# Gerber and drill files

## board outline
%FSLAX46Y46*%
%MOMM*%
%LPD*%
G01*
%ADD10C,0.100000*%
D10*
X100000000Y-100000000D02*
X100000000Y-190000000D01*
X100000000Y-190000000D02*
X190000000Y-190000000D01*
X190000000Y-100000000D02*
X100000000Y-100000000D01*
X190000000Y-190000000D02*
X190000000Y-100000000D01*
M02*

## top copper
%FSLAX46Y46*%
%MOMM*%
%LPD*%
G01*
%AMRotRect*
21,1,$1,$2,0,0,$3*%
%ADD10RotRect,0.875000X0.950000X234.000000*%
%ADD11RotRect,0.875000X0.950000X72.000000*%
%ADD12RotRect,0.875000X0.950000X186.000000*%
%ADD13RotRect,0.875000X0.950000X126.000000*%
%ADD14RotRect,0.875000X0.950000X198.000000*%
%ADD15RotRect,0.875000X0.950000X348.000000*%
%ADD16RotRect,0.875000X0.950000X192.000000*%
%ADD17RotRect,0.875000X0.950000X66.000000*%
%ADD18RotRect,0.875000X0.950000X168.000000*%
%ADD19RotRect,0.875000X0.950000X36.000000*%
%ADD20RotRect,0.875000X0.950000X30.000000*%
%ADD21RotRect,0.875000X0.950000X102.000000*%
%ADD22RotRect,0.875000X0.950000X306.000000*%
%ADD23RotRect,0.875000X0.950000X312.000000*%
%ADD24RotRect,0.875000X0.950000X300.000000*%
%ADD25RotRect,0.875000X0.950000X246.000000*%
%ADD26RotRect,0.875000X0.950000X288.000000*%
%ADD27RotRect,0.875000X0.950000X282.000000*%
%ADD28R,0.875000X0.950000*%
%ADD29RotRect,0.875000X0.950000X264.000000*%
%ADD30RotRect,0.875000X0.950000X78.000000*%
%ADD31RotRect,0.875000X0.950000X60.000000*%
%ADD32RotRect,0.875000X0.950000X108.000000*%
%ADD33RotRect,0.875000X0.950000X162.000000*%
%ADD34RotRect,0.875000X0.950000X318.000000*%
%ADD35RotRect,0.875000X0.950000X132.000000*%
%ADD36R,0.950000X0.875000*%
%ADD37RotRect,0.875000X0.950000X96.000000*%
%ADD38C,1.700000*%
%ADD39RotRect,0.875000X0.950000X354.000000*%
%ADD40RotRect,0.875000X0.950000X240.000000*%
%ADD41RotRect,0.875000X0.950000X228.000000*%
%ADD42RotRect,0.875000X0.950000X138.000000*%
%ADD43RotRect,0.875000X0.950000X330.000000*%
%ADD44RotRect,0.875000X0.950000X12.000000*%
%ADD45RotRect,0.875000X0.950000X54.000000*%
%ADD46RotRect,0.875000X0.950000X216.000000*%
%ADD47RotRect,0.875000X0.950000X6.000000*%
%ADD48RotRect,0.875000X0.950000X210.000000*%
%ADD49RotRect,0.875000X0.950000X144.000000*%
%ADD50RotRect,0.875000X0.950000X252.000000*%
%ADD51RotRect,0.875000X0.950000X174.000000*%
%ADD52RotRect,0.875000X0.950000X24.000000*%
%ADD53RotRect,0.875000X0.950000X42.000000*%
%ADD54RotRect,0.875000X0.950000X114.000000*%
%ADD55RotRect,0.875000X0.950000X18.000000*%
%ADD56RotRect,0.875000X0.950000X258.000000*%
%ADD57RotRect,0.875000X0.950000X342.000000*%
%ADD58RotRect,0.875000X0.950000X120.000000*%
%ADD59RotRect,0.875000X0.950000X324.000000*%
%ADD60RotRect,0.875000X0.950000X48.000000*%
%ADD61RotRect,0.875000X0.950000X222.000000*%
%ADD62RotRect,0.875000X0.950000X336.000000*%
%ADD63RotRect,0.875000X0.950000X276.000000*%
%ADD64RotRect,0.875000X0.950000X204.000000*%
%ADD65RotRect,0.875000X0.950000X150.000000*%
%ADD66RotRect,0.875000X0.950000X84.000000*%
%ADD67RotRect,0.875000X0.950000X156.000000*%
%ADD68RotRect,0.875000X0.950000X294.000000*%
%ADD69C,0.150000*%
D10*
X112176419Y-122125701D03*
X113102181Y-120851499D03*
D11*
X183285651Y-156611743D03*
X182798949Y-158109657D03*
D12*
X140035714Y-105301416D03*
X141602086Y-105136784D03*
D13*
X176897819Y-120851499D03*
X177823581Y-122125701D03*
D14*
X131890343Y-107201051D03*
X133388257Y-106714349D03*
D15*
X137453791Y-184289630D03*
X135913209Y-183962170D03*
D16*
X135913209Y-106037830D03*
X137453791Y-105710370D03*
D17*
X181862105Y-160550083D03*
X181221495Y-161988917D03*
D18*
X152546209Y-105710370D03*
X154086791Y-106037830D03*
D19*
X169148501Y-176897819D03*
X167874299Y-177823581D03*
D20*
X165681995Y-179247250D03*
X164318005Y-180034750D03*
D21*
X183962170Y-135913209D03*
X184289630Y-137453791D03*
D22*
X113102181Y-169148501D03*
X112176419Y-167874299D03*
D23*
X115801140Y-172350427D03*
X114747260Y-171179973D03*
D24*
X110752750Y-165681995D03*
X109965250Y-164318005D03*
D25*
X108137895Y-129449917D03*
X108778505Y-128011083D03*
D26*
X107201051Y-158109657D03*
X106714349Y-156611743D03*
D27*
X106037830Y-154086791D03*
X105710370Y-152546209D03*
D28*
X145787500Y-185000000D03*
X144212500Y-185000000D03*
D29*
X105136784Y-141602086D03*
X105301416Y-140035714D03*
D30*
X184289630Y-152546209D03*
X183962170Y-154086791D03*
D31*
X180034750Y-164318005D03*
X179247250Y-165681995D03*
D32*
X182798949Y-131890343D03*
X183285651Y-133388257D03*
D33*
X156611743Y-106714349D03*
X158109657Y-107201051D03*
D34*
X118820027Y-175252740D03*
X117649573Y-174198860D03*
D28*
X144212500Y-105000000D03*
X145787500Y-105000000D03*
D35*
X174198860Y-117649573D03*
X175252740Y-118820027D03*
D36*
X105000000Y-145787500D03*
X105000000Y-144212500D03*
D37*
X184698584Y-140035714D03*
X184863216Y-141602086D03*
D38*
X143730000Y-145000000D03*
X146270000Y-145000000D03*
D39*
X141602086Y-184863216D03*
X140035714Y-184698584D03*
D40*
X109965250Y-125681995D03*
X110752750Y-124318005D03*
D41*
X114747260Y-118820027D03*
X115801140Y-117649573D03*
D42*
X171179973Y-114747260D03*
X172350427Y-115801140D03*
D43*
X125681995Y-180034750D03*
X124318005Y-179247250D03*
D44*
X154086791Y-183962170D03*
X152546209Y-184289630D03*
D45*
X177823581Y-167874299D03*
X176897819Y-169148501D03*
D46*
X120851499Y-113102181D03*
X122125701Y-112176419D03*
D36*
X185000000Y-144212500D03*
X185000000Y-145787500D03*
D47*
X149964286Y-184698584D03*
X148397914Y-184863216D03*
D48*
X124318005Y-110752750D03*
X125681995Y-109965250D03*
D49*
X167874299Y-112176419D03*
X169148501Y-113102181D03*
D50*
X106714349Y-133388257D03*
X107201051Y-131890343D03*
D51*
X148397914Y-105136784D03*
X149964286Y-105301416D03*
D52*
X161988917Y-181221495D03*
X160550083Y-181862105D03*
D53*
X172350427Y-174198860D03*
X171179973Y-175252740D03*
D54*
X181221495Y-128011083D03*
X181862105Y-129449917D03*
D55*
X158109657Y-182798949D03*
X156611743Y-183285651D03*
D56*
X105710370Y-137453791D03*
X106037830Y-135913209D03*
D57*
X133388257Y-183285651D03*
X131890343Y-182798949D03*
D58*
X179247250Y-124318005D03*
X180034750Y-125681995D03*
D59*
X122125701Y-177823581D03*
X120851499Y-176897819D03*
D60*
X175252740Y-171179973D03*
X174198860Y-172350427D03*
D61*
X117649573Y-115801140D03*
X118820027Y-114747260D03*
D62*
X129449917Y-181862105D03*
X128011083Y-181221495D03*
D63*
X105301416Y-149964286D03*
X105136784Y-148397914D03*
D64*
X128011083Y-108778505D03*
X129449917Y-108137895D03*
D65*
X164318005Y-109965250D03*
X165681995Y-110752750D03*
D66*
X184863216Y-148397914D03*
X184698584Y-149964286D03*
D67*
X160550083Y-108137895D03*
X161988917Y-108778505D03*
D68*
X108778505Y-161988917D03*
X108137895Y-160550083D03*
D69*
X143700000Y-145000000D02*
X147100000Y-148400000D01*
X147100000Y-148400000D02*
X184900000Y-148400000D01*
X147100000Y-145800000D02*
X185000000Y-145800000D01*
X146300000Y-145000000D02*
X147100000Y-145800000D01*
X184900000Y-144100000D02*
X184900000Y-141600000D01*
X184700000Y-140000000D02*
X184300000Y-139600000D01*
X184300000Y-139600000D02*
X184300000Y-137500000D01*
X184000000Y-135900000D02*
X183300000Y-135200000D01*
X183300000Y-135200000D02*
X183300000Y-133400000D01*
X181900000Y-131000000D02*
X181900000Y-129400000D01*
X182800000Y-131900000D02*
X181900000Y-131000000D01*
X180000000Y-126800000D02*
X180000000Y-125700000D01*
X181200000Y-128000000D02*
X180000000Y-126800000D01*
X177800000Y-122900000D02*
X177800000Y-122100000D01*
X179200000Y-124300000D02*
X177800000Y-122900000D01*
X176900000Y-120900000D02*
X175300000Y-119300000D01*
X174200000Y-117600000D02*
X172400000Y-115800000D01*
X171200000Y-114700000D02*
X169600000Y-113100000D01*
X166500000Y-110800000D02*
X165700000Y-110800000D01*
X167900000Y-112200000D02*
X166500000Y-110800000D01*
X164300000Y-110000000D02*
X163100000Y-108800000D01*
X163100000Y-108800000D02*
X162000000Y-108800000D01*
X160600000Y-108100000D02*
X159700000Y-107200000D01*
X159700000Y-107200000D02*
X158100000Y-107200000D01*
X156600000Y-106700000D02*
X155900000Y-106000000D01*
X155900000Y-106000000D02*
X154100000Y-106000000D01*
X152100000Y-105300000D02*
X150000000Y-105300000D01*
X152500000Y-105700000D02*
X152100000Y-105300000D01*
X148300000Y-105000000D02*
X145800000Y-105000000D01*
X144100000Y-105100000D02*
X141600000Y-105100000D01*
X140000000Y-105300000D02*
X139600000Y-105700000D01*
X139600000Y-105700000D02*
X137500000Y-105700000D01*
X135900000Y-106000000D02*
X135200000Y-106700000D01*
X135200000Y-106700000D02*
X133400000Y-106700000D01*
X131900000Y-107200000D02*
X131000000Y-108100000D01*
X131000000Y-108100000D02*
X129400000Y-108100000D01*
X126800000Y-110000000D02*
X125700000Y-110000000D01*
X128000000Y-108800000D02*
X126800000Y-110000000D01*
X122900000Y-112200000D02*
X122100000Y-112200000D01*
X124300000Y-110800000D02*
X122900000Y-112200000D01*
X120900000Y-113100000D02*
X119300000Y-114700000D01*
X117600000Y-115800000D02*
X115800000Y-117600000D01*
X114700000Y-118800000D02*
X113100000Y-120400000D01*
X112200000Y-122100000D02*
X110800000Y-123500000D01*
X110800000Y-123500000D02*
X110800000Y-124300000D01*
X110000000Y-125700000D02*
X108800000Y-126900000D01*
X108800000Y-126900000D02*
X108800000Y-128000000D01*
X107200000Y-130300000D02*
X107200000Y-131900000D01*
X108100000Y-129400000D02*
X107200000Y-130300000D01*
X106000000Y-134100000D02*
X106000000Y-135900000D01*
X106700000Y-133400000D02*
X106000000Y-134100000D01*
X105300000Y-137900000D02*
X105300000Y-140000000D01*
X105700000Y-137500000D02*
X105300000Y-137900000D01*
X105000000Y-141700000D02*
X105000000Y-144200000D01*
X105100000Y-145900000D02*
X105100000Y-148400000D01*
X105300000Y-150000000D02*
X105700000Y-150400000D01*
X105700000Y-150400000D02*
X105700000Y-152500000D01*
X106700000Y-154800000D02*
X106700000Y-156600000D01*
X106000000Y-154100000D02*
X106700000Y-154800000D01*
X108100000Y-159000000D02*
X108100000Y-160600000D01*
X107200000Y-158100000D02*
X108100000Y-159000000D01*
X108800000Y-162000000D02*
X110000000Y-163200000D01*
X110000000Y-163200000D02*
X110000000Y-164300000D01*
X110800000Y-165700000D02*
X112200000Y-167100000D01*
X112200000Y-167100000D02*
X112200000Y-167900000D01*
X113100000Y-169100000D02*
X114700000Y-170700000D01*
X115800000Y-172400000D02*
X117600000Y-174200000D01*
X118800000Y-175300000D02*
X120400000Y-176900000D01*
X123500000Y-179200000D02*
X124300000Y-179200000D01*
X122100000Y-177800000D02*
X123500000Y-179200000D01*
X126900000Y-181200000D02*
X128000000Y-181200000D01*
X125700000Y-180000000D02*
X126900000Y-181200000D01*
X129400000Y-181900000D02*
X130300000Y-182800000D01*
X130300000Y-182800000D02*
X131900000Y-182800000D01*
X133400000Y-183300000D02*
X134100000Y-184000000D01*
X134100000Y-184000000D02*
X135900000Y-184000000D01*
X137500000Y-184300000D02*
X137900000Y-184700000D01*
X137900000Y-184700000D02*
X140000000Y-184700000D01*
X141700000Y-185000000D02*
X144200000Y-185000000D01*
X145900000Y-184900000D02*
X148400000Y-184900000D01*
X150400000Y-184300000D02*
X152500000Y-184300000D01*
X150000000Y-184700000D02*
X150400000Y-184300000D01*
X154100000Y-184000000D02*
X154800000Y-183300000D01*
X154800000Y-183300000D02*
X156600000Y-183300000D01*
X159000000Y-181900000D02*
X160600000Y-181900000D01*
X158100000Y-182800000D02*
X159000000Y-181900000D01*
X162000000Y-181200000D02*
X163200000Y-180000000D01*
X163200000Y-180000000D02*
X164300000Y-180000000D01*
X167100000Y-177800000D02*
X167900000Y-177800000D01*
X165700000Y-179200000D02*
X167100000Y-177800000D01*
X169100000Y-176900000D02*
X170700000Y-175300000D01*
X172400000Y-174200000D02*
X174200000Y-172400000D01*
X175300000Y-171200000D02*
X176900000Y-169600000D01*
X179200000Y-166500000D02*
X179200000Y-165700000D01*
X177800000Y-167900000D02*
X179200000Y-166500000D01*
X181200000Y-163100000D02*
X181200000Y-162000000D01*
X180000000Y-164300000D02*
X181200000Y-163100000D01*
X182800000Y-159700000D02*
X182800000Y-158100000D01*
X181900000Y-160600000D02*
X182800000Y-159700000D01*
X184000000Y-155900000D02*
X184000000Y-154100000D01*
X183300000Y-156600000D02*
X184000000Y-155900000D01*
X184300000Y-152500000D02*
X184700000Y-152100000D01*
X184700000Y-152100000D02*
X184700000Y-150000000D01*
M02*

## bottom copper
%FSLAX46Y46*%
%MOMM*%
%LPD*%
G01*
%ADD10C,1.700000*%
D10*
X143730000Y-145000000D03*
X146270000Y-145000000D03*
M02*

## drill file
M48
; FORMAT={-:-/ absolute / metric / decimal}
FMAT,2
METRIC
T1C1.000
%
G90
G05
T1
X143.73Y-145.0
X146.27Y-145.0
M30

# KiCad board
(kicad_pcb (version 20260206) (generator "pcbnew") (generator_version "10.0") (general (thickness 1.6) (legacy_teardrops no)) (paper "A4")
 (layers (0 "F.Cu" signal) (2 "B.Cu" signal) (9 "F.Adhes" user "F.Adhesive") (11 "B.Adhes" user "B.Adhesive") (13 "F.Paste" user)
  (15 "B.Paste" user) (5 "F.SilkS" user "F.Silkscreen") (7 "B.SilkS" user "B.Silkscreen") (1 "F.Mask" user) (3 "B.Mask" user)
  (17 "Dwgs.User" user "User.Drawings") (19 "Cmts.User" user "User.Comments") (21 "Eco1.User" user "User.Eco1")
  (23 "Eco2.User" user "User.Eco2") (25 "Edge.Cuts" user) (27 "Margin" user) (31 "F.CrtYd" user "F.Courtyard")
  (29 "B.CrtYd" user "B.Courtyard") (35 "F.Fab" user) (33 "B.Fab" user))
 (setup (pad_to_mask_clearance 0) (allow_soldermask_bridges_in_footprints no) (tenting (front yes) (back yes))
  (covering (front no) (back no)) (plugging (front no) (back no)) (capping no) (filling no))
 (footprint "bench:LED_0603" (layer "F.Cu") (at 112.6393 121.4886 -126)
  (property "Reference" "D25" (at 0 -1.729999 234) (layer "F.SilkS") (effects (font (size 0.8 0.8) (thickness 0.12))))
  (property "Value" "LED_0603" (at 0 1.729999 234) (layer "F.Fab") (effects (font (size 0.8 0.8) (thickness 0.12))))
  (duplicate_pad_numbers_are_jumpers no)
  (pad "A" smd rect (at 0.7875 0 234) (size 0.875 0.95) (layers "F.Cu" "F.Mask" "F.Paste") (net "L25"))
  (pad "K" smd rect (at -0.7875 0 234) (size 0.875 0.95) (layers "F.Cu" "F.Mask" "F.Paste") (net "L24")))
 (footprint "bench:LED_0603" (layer "F.Cu") (at 183.0423 157.3607 72)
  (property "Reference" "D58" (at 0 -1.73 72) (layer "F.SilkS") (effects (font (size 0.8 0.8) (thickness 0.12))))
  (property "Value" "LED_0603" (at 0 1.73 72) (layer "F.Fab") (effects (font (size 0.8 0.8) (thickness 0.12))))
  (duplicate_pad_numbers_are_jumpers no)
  (pad "A" smd rect (at 0.7875 0 72) (size 0.875 0.95) (layers "F.Cu" "F.Mask" "F.Paste") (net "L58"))
  (pad "K" smd rect (at -0.7875 0 72) (size 0.875 0.95) (layers "F.Cu" "F.Mask" "F.Paste") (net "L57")))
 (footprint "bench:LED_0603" (layer "F.Cu") (at 140.8189 105.2191 -174)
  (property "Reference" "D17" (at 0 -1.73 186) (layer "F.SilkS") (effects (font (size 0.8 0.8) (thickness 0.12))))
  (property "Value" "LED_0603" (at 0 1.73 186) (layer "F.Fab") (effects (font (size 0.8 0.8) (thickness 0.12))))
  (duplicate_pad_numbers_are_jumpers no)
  (pad "A" smd rect (at 0.7875 0 186) (size 0.875 0.95) (layers "F.Cu" "F.Mask" "F.Paste") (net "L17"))
  (pad "K" smd rect (at -0.7875 0 186) (size 0.875 0.95) (layers "F.Cu" "F.Mask" "F.Paste") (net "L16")))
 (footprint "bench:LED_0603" (layer "F.Cu") (at 177.3607 121.4886 126)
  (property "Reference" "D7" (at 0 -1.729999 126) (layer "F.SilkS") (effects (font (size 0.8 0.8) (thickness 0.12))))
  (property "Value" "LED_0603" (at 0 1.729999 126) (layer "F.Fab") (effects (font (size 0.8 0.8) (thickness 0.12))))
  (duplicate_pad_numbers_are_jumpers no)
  (pad "A" smd rect (at 0.7875 0 126) (size 0.875 0.95) (layers "F.Cu" "F.Mask" "F.Paste") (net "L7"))
  (pad "K" smd rect (at -0.7875 0 126) (size 0.875 0.95) (layers "F.Cu" "F.Mask" "F.Paste") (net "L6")))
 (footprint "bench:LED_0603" (layer "F.Cu") (at 132.6393 106.9577 -162)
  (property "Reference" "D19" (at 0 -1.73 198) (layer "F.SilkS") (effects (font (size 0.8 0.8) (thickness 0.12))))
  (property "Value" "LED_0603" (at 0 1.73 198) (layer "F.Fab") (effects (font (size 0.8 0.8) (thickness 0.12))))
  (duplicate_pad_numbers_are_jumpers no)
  (pad "A" smd rect (at 0.7875 0 198) (size 0.875 0.95) (layers "F.Cu" "F.Mask" "F.Paste") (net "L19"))
  (pad "K" smd rect (at -0.7875 0 198) (size 0.875 0.95) (layers "F.Cu" "F.Mask" "F.Paste") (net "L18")))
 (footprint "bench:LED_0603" (layer "F.Cu") (at 136.6835 184.1259 -12)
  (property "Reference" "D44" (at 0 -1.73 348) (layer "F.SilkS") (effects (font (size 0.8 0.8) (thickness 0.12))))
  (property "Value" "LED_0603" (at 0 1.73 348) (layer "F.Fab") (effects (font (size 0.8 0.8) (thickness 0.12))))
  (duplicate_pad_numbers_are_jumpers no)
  (pad "A" smd rect (at 0.7875 0 348) (size 0.875 0.95) (layers "F.Cu" "F.Mask" "F.Paste") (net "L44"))
  (pad "K" smd rect (at -0.7875 0 348) (size 0.875 0.95) (layers "F.Cu" "F.Mask" "F.Paste") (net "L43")))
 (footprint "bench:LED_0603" (layer "F.Cu") (at 136.6835 105.8741 -168)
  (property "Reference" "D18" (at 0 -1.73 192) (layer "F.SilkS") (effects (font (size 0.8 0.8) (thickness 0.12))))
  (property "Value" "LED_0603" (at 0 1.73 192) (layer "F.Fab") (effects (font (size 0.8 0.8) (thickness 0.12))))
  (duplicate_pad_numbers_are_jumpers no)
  (pad "A" smd rect (at 0.7875 0 192) (size 0.875 0.95) (layers "F.Cu" "F.Mask" "F.Paste") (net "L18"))
  (pad "K" smd rect (at -0.7875 0 192) (size 0.875 0.95) (layers "F.Cu" "F.Mask" "F.Paste") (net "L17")))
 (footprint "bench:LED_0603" (layer "F.Cu") (at 181.5418 161.2695 66)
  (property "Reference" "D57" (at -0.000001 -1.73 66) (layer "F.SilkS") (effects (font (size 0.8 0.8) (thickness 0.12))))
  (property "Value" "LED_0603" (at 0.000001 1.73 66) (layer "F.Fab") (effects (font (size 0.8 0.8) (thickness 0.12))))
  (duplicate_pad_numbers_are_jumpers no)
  (pad "A" smd rect (at 0.7875 0 66) (size 0.875 0.95) (layers "F.Cu" "F.Mask" "F.Paste") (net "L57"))
  (pad "K" smd rect (at -0.7875 0 66) (size 0.875 0.95) (layers "F.Cu" "F.Mask" "F.Paste") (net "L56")))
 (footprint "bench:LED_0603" (layer "F.Cu") (at 153.3165 105.8741 168)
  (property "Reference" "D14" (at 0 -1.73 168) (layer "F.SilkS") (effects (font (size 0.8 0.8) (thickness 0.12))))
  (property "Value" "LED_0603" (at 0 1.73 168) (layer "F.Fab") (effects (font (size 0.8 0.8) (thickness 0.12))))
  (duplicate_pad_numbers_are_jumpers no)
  (pad "A" smd rect (at 0.7875 0 168) (size 0.875 0.95) (layers "F.Cu" "F.Mask" "F.Paste") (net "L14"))
  (pad "K" smd rect (at -0.7875 0 168) (size 0.875 0.95) (layers "F.Cu" "F.Mask" "F.Paste") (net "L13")))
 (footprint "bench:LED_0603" (layer "F.Cu") (at 168.5114 177.3607 36)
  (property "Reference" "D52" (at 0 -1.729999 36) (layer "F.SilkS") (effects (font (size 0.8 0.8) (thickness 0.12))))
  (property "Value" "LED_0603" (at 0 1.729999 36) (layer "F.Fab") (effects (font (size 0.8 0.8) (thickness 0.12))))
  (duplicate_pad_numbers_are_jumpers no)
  (pad "A" smd rect (at 0.7875 0 36) (size 0.875 0.95) (layers "F.Cu" "F.Mask" "F.Paste") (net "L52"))
  (pad "K" smd rect (at -0.7875 0 36) (size 0.875 0.95) (layers "F.Cu" "F.Mask" "F.Paste") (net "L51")))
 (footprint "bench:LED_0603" (layer "F.Cu") (at 165 179.641 30)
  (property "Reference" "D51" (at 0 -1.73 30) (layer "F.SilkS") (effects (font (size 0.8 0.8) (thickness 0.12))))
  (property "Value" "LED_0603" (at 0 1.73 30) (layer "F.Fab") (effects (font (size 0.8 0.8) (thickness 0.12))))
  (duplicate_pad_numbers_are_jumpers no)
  (pad "A" smd rect (at 0.7875 0 30) (size 0.875 0.95) (layers "F.Cu" "F.Mask" "F.Paste") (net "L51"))
  (pad "K" smd rect (at -0.7875 0 30) (size 0.875 0.95) (layers "F.Cu" "F.Mask" "F.Paste") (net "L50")))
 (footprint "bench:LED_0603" (layer "F.Cu") (at 184.1259 136.6835 102)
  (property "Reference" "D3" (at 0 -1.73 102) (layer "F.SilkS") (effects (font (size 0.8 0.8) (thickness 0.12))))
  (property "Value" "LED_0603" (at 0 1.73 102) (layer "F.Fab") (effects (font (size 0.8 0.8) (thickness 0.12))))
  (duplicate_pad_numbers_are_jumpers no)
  (pad "A" smd rect (at 0.7875 0 102) (size 0.875 0.95) (layers "F.Cu" "F.Mask" "F.Paste") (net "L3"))
  (pad "K" smd rect (at -0.7875 0 102) (size 0.875 0.95) (layers "F.Cu" "F.Mask" "F.Paste") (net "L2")))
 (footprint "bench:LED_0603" (layer "F.Cu") (at 112.6393 168.5114 -54)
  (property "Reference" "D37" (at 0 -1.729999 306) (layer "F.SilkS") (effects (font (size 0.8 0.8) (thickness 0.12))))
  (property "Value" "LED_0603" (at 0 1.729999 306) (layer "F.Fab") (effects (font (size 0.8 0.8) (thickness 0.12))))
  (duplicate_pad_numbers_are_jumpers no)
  (pad "A" smd rect (at 0.7875 0 306) (size 0.875 0.95) (layers "F.Cu" "F.Mask" "F.Paste") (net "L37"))
  (pad "K" smd rect (at -0.7875 0 306) (size 0.875 0.95) (layers "F.Cu" "F.Mask" "F.Paste") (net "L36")))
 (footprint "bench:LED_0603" (layer "F.Cu") (at 115.2742 171.7652 -48)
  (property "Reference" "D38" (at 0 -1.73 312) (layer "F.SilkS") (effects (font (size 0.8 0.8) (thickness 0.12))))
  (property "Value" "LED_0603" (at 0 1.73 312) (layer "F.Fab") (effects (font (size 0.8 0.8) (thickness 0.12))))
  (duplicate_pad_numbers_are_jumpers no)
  (pad "A" smd rect (at 0.7875 0.000001 312) (size 0.875 0.95) (layers "F.Cu" "F.Mask" "F.Paste") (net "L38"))
  (pad "K" smd rect (at -0.7875 -0.000001 312) (size 0.875 0.95) (layers "F.Cu" "F.Mask" "F.Paste") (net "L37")))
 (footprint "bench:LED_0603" (layer "F.Cu") (at 110.359 165 -60)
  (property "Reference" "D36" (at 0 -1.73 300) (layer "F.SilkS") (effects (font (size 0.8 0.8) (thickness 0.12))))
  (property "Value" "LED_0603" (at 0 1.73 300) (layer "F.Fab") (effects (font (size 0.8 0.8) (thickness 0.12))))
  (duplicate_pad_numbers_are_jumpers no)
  (pad "A" smd rect (at 0.7875 0 300) (size 0.875 0.95) (layers "F.Cu" "F.Mask" "F.Paste") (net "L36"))
  (pad "K" smd rect (at -0.7875 0 300) (size 0.875 0.95) (layers "F.Cu" "F.Mask" "F.Paste") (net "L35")))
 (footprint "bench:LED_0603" (layer "F.Cu") (at 108.4582 128.7305 -114)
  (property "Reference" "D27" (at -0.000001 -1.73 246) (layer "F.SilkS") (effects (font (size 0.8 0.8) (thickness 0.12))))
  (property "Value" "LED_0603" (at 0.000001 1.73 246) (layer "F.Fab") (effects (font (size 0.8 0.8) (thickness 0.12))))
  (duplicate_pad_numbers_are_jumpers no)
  (pad "A" smd rect (at 0.7875 0 246) (size 0.875 0.95) (layers "F.Cu" "F.Mask" "F.Paste") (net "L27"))
  (pad "K" smd rect (at -0.7875 0 246) (size 0.875 0.95) (layers "F.Cu" "F.Mask" "F.Paste") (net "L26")))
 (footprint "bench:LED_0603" (layer "F.Cu") (at 106.9577 157.3607 -72)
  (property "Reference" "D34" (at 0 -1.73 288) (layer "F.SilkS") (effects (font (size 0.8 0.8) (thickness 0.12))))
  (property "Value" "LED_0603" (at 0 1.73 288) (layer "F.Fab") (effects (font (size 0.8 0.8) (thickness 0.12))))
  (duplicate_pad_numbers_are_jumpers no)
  (pad "A" smd rect (at 0.7875 0 288) (size 0.875 0.95) (layers "F.Cu" "F.Mask" "F.Paste") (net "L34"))
  (pad "K" smd rect (at -0.7875 0 288) (size 0.875 0.95) (layers "F.Cu" "F.Mask" "F.Paste") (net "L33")))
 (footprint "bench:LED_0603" (layer "F.Cu") (at 105.8741 153.3165 -78)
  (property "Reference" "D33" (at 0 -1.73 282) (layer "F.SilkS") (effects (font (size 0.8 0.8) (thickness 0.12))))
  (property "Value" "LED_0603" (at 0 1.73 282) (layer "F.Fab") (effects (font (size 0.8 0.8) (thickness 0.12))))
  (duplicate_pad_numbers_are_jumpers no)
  (pad "A" smd rect (at 0.7875 0 282) (size 0.875 0.95) (layers "F.Cu" "F.Mask" "F.Paste") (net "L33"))
  (pad "K" smd rect (at -0.7875 0 282) (size 0.875 0.95) (layers "F.Cu" "F.Mask" "F.Paste") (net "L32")))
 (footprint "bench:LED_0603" (layer "F.Cu") (at 145 185)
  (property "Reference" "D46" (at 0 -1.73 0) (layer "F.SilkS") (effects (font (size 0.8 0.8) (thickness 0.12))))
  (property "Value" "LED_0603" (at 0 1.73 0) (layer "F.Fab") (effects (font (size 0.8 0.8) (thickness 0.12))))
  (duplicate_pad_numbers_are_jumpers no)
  (pad "A" smd rect (at 0.7875 0) (size 0.875 0.95) (layers "F.Cu" "F.Mask" "F.Paste") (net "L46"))
  (pad "K" smd rect (at -0.7875 0) (size 0.875 0.95) (layers "F.Cu" "F.Mask" "F.Paste") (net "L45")))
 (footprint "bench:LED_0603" (layer "F.Cu") (at 105.2191 140.8189 -96)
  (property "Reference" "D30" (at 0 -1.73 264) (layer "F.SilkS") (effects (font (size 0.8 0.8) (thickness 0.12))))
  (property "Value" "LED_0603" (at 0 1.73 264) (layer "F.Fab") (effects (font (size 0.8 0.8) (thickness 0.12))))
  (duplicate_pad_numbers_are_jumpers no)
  (pad "A" smd rect (at 0.7875 0 264) (size 0.875 0.95) (layers "F.Cu" "F.Mask" "F.Paste") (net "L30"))
  (pad "K" smd rect (at -0.7875 0 264) (size 0.875 0.95) (layers "F.Cu" "F.Mask" "F.Paste") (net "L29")))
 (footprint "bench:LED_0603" (layer "F.Cu") (at 184.1259 153.3165 78)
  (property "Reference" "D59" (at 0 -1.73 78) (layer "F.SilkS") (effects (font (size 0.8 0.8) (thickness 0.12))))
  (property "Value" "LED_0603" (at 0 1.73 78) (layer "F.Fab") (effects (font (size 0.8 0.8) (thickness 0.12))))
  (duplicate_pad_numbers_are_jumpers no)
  (pad "A" smd rect (at 0.7875 0 78) (size 0.875 0.95) (layers "F.Cu" "F.Mask" "F.Paste") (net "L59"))
  (pad "K" smd rect (at -0.7875 0 78) (size 0.875 0.95) (layers "F.Cu" "F.Mask" "F.Paste") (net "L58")))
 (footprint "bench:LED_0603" (layer "F.Cu") (at 179.641 165 60)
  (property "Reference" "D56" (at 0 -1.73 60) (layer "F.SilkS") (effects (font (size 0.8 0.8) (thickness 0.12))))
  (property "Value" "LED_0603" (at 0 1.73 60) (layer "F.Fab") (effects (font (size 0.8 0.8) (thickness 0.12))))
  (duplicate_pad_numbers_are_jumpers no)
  (pad "A" smd rect (at 0.7875 0 60) (size 0.875 0.95) (layers "F.Cu" "F.Mask" "F.Paste") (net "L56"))
  (pad "K" smd rect (at -0.7875 0 60) (size 0.875 0.95) (layers "F.Cu" "F.Mask" "F.Paste") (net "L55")))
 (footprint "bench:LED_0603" (layer "F.Cu") (at 183.0423 132.6393 108)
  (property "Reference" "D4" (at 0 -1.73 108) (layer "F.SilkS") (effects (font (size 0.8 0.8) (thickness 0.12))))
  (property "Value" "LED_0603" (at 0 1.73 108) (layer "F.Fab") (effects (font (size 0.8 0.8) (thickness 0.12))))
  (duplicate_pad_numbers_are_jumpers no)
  (pad "A" smd rect (at 0.7875 0 108) (size 0.875 0.95) (layers "F.Cu" "F.Mask" "F.Paste") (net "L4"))
  (pad "K" smd rect (at -0.7875 0 108) (size 0.875 0.95) (layers "F.Cu" "F.Mask" "F.Paste") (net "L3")))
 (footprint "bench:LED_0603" (layer "F.Cu") (at 157.3607 106.9577 162)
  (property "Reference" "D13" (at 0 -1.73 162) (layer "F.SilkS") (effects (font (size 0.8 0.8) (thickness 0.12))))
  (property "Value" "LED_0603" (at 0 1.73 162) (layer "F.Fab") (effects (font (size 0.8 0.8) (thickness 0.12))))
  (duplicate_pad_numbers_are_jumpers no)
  (pad "A" smd rect (at 0.7875 0 162) (size 0.875 0.95) (layers "F.Cu" "F.Mask" "F.Paste") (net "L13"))
  (pad "K" smd rect (at -0.7875 0 162) (size 0.875 0.95) (layers "F.Cu" "F.Mask" "F.Paste") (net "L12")))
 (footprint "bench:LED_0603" (layer "F.Cu") (at 118.2348 174.7258 -42)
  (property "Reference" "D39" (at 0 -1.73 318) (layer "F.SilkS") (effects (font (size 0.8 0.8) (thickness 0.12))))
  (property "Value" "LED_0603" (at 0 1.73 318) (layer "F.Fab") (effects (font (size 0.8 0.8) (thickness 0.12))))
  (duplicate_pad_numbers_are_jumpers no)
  (pad "A" smd rect (at 0.7875 -0.000001 318) (size 0.875 0.95) (layers "F.Cu" "F.Mask" "F.Paste") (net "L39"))
  (pad "K" smd rect (at -0.7875 0.000001 318) (size 0.875 0.95) (layers "F.Cu" "F.Mask" "F.Paste") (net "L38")))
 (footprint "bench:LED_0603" (layer "F.Cu") (at 145 105 180)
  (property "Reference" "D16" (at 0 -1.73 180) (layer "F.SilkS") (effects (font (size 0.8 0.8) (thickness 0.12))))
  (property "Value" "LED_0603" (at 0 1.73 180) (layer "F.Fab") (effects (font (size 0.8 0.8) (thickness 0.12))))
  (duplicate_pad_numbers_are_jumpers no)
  (pad "A" smd rect (at 0.7875 0 180) (size 0.875 0.95) (layers "F.Cu" "F.Mask" "F.Paste") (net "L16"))
  (pad "K" smd rect (at -0.7875 0 180) (size 0.875 0.95) (layers "F.Cu" "F.Mask" "F.Paste") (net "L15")))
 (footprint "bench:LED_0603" (layer "F.Cu") (at 174.7258 118.2348 132)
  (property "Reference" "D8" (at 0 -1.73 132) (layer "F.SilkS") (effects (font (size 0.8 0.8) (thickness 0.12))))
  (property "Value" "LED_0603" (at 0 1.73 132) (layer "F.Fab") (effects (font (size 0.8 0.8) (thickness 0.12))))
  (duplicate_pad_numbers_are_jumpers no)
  (pad "A" smd rect (at 0.7875 0.000001 132) (size 0.875 0.95) (layers "F.Cu" "F.Mask" "F.Paste") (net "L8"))
  (pad "K" smd rect (at -0.7875 -0.000001 132) (size 0.875 0.95) (layers "F.Cu" "F.Mask" "F.Paste") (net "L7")))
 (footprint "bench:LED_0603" (layer "F.Cu") (at 105 145 -90)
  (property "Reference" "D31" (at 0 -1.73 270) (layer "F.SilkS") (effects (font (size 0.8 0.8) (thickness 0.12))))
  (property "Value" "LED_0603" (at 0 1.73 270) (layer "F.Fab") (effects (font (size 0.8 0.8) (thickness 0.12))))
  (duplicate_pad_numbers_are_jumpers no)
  (pad "A" smd rect (at 0.7875 0 270) (size 0.875 0.95) (layers "F.Cu" "F.Mask" "F.Paste") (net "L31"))
  (pad "K" smd rect (at -0.7875 0 270) (size 0.875 0.95) (layers "F.Cu" "F.Mask" "F.Paste") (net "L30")))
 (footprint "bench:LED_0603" (layer "F.Cu") (at 184.7809 140.8189 96)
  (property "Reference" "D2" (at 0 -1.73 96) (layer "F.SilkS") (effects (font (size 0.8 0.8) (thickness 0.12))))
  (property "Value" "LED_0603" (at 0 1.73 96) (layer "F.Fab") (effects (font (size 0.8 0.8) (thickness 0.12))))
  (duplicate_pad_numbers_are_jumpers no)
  (pad "A" smd rect (at 0.7875 0 96) (size 0.875 0.95) (layers "F.Cu" "F.Mask" "F.Paste") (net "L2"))
  (pad "K" smd rect (at -0.7875 0 96) (size 0.875 0.95) (layers "F.Cu" "F.Mask" "F.Paste") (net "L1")))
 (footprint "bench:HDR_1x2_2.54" (layer "F.Cu") (at 143.73 145)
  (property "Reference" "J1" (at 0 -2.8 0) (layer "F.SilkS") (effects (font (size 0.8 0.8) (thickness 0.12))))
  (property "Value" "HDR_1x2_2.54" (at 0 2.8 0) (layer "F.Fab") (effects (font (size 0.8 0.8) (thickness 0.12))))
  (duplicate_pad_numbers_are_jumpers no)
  (pad "1" thru_hole circle (at 0 0) (size 1.7 1.7) (drill 1) (layers "*.Cu" "*.Mask") (remove_unused_layers no) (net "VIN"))
  (pad "2" thru_hole circle (at 2.54 0) (size 1.7 1.7) (drill 1) (layers "*.Cu" "*.Mask") (remove_unused_layers no) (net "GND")))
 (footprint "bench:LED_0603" (layer "F.Cu") (at 140.8189 184.7809 -6)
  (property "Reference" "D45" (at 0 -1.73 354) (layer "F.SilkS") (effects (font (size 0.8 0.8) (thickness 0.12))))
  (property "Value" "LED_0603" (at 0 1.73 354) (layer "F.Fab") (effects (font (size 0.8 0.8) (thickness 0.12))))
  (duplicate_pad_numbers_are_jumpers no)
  (pad "A" smd rect (at 0.7875 0 354) (size 0.875 0.95) (layers "F.Cu" "F.Mask" "F.Paste") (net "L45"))
  (pad "K" smd rect (at -0.7875 0 354) (size 0.875 0.95) (layers "F.Cu" "F.Mask" "F.Paste") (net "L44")))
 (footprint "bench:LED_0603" (layer "F.Cu") (at 110.359 125 -120)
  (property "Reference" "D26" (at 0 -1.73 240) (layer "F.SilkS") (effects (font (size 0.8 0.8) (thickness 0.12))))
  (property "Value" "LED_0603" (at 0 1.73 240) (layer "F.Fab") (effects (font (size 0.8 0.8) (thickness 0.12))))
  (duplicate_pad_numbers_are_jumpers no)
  (pad "A" smd rect (at 0.7875 0 240) (size 0.875 0.95) (layers "F.Cu" "F.Mask" "F.Paste") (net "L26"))
  (pad "K" smd rect (at -0.7875 0 240) (size 0.875 0.95) (layers "F.Cu" "F.Mask" "F.Paste") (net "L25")))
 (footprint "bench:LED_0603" (layer "F.Cu") (at 115.2742 118.2348 -132)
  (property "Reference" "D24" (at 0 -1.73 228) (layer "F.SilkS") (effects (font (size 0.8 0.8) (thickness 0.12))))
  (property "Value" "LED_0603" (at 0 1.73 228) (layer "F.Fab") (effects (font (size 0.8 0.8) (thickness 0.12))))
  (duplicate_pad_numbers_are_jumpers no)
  (pad "A" smd rect (at 0.7875 -0.000001 228) (size 0.875 0.95) (layers "F.Cu" "F.Mask" "F.Paste") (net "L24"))
  (pad "K" smd rect (at -0.7875 0.000001 228) (size 0.875 0.95) (layers "F.Cu" "F.Mask" "F.Paste") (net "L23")))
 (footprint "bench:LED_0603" (layer "F.Cu") (at 171.7652 115.2742 138)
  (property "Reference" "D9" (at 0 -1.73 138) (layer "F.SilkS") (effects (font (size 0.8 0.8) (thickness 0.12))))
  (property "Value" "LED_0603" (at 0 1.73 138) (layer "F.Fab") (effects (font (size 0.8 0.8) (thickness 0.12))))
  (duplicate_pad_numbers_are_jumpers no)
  (pad "A" smd rect (at 0.7875 -0.000001 138) (size 0.875 0.95) (layers "F.Cu" "F.Mask" "F.Paste") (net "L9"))
  (pad "K" smd rect (at -0.7875 0.000001 138) (size 0.875 0.95) (layers "F.Cu" "F.Mask" "F.Paste") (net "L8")))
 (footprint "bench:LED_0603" (layer "F.Cu") (at 125 179.641 -30)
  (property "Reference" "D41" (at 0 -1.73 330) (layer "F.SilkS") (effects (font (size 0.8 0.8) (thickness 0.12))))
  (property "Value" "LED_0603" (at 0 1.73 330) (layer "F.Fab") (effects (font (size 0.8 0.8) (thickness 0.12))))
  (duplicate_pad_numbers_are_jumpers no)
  (pad "A" smd rect (at 0.7875 0 330) (size 0.875 0.95) (layers "F.Cu" "F.Mask" "F.Paste") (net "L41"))
  (pad "K" smd rect (at -0.7875 0 330) (size 0.875 0.95) (layers "F.Cu" "F.Mask" "F.Paste") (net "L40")))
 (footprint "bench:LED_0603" (layer "F.Cu") (at 153.3165 184.1259 12)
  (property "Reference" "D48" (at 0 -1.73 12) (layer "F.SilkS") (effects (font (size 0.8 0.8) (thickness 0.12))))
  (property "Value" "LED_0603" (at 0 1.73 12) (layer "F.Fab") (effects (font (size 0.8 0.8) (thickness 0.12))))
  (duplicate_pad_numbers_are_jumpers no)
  (pad "A" smd rect (at 0.7875 0 12) (size 0.875 0.95) (layers "F.Cu" "F.Mask" "F.Paste") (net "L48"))
  (pad "K" smd rect (at -0.7875 0 12) (size 0.875 0.95) (layers "F.Cu" "F.Mask" "F.Paste") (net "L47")))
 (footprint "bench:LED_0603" (layer "F.Cu") (at 177.3607 168.5114 54)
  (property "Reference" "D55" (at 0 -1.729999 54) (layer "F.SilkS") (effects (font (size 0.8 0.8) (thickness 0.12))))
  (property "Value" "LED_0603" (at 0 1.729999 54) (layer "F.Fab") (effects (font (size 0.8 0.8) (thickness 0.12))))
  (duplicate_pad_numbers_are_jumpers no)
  (pad "A" smd rect (at 0.7875 0 54) (size 0.875 0.95) (layers "F.Cu" "F.Mask" "F.Paste") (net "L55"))
  (pad "K" smd rect (at -0.7875 0 54) (size 0.875 0.95) (layers "F.Cu" "F.Mask" "F.Paste") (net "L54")))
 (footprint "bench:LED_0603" (layer "F.Cu") (at 121.4886 112.6393 -144)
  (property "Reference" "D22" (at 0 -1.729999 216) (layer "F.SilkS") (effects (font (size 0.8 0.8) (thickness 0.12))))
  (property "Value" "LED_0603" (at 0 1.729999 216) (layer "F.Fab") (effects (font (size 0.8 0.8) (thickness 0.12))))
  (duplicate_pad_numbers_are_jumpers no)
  (pad "A" smd rect (at 0.7875 0 216) (size 0.875 0.95) (layers "F.Cu" "F.Mask" "F.Paste") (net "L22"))
  (pad "K" smd rect (at -0.7875 0 216) (size 0.875 0.95) (layers "F.Cu" "F.Mask" "F.Paste") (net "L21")))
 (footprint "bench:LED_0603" (layer "F.Cu") (at 185 145 90)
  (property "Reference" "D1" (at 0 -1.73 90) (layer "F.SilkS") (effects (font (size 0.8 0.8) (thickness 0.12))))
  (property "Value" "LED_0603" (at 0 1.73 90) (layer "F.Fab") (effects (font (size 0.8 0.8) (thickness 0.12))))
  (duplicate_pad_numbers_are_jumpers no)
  (pad "A" smd rect (at 0.7875 0 90) (size 0.875 0.95) (layers "F.Cu" "F.Mask" "F.Paste") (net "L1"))
  (pad "K" smd rect (at -0.7875 0 90) (size 0.875 0.95) (layers "F.Cu" "F.Mask" "F.Paste") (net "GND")))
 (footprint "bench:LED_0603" (layer "F.Cu") (at 149.1811 184.7809 6)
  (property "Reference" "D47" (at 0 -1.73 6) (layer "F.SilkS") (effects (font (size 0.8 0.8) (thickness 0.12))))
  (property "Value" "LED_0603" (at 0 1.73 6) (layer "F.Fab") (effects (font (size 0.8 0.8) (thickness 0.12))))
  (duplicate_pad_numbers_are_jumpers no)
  (pad "A" smd rect (at 0.7875 0 6) (size 0.875 0.95) (layers "F.Cu" "F.Mask" "F.Paste") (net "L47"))
  (pad "K" smd rect (at -0.7875 0 6) (size 0.875 0.95) (layers "F.Cu" "F.Mask" "F.Paste") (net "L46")))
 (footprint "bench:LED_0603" (layer "F.Cu") (at 125 110.359 -150)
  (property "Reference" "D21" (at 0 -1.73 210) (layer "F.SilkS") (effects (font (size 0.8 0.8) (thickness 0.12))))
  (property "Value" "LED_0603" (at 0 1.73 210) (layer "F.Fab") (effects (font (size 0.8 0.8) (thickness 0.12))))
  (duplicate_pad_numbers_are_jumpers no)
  (pad "A" smd rect (at 0.7875 0 210) (size 0.875 0.95) (layers "F.Cu" "F.Mask" "F.Paste") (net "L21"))
  (pad "K" smd rect (at -0.7875 0 210) (size 0.875 0.95) (layers "F.Cu" "F.Mask" "F.Paste") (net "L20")))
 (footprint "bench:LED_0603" (layer "F.Cu") (at 168.5114 112.6393 144)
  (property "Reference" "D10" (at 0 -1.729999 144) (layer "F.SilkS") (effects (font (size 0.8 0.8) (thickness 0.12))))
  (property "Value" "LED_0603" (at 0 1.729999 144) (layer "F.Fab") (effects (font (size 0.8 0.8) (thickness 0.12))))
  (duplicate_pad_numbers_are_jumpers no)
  (pad "A" smd rect (at 0.7875 0 144) (size 0.875 0.95) (layers "F.Cu" "F.Mask" "F.Paste") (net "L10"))
  (pad "K" smd rect (at -0.7875 0 144) (size 0.875 0.95) (layers "F.Cu" "F.Mask" "F.Paste") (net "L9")))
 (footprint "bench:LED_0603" (layer "F.Cu") (at 106.9577 132.6393 -108)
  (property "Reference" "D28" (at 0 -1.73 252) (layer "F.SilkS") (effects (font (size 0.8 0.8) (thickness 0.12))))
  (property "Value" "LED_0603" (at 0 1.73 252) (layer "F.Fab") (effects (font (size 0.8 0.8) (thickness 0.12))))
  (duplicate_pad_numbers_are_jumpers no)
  (pad "A" smd rect (at 0.7875 0 252) (size 0.875 0.95) (layers "F.Cu" "F.Mask" "F.Paste") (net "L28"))
  (pad "K" smd rect (at -0.7875 0 252) (size 0.875 0.95) (layers "F.Cu" "F.Mask" "F.Paste") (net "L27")))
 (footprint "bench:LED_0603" (layer "F.Cu") (at 149.1811 105.2191 174)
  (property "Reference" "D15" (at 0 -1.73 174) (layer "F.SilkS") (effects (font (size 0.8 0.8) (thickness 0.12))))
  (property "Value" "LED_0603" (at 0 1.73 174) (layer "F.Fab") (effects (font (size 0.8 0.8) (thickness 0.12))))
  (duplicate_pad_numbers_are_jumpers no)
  (pad "A" smd rect (at 0.7875 0 174) (size 0.875 0.95) (layers "F.Cu" "F.Mask" "F.Paste") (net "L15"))
  (pad "K" smd rect (at -0.7875 0 174) (size 0.875 0.95) (layers "F.Cu" "F.Mask" "F.Paste") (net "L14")))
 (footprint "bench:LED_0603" (layer "F.Cu") (at 161.2695 181.5418 24)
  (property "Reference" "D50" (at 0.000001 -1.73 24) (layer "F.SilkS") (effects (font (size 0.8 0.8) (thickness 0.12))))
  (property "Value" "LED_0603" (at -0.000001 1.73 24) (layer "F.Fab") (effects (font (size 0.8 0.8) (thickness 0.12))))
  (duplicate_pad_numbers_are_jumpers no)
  (pad "A" smd rect (at 0.7875 0 24) (size 0.875 0.95) (layers "F.Cu" "F.Mask" "F.Paste") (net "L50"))
  (pad "K" smd rect (at -0.7875 0 24) (size 0.875 0.95) (layers "F.Cu" "F.Mask" "F.Paste") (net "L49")))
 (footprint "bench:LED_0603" (layer "F.Cu") (at 171.7652 174.7258 42)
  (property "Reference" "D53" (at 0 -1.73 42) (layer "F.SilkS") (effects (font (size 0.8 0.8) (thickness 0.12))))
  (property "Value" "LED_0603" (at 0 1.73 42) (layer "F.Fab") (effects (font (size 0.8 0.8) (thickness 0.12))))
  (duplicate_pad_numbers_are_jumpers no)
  (pad "A" smd rect (at 0.7875 0.000001 42) (size 0.875 0.95) (layers "F.Cu" "F.Mask" "F.Paste") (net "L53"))
  (pad "K" smd rect (at -0.7875 -0.000001 42) (size 0.875 0.95) (layers "F.Cu" "F.Mask" "F.Paste") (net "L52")))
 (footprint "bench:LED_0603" (layer "F.Cu") (at 181.5418 128.7305 114)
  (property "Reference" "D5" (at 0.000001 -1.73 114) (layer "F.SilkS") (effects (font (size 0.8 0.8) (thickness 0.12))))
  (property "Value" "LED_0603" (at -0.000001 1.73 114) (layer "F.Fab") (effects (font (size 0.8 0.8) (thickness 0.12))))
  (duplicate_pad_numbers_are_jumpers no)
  (pad "A" smd rect (at 0.7875 0 114) (size 0.875 0.95) (layers "F.Cu" "F.Mask" "F.Paste") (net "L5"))
  (pad "K" smd rect (at -0.7875 0 114) (size 0.875 0.95) (layers "F.Cu" "F.Mask" "F.Paste") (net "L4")))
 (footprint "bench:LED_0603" (layer "F.Cu") (at 157.3607 183.0423 18)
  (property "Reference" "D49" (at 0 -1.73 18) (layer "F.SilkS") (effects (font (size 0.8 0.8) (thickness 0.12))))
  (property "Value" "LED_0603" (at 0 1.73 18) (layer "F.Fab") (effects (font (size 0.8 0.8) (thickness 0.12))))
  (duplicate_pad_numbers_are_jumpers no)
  (pad "A" smd rect (at 0.7875 0 18) (size 0.875 0.95) (layers "F.Cu" "F.Mask" "F.Paste") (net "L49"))
  (pad "K" smd rect (at -0.7875 0 18) (size 0.875 0.95) (layers "F.Cu" "F.Mask" "F.Paste") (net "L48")))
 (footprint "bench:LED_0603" (layer "F.Cu") (at 105.8741 136.6835 -102)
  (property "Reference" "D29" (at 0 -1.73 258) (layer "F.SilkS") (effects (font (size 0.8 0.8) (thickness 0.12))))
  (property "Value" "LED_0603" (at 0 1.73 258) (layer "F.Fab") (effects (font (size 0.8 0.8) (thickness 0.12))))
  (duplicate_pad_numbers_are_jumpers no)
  (pad "A" smd rect (at 0.7875 0 258) (size 0.875 0.95) (layers "F.Cu" "F.Mask" "F.Paste") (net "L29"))
  (pad "K" smd rect (at -0.7875 0 258) (size 0.875 0.95) (layers "F.Cu" "F.Mask" "F.Paste") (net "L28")))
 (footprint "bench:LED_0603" (layer "F.Cu") (at 132.6393 183.0423 -18)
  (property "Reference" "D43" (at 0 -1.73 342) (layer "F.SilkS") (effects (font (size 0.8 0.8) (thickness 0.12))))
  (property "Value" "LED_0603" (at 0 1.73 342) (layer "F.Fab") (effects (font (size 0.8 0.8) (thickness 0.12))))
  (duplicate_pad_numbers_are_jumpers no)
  (pad "A" smd rect (at 0.7875 0 342) (size 0.875 0.95) (layers "F.Cu" "F.Mask" "F.Paste") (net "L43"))
  (pad "K" smd rect (at -0.7875 0 342) (size 0.875 0.95) (layers "F.Cu" "F.Mask" "F.Paste") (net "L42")))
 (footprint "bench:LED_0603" (layer "F.Cu") (at 179.641 125 120)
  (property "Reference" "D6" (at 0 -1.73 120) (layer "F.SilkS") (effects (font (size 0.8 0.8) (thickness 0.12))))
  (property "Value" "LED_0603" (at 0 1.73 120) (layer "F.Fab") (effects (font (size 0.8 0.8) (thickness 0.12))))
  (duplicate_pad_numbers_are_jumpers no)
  (pad "A" smd rect (at 0.7875 0 120) (size 0.875 0.95) (layers "F.Cu" "F.Mask" "F.Paste") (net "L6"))
  (pad "K" smd rect (at -0.7875 0 120) (size 0.875 0.95) (layers "F.Cu" "F.Mask" "F.Paste") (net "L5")))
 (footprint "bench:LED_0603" (layer "F.Cu") (at 121.4886 177.3607 -36)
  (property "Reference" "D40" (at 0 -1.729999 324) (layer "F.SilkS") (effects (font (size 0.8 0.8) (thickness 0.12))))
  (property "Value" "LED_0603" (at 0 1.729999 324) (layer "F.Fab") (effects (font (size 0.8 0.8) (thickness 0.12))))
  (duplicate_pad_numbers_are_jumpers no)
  (pad "A" smd rect (at 0.7875 0 324) (size 0.875 0.95) (layers "F.Cu" "F.Mask" "F.Paste") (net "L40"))
  (pad "K" smd rect (at -0.7875 0 324) (size 0.875 0.95) (layers "F.Cu" "F.Mask" "F.Paste") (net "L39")))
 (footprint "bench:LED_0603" (layer "F.Cu") (at 174.7258 171.7652 48)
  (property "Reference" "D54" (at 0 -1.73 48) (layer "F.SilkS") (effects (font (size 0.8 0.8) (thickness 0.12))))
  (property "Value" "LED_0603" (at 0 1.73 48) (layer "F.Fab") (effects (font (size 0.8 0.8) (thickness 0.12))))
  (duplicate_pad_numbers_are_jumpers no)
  (pad "A" smd rect (at 0.7875 -0.000001 48) (size 0.875 0.95) (layers "F.Cu" "F.Mask" "F.Paste") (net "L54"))
  (pad "K" smd rect (at -0.7875 0.000001 48) (size 0.875 0.95) (layers "F.Cu" "F.Mask" "F.Paste") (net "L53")))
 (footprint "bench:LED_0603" (layer "F.Cu") (at 118.2348 115.2742 -138)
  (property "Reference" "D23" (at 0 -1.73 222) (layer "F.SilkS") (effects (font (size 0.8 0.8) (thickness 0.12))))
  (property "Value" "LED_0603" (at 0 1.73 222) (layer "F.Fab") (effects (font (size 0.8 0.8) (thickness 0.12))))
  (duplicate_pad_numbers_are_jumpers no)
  (pad "A" smd rect (at 0.7875 0.000001 222) (size 0.875 0.95) (layers "F.Cu" "F.Mask" "F.Paste") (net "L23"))
  (pad "K" smd rect (at -0.7875 -0.000001 222) (size 0.875 0.95) (layers "F.Cu" "F.Mask" "F.Paste") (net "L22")))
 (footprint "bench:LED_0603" (layer "F.Cu") (at 128.7305 181.5418 -24)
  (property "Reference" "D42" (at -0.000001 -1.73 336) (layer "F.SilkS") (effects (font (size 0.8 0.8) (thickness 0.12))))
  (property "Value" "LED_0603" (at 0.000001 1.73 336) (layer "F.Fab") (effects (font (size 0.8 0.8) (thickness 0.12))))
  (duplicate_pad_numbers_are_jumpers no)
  (pad "A" smd rect (at 0.7875 0 336) (size 0.875 0.95) (layers "F.Cu" "F.Mask" "F.Paste") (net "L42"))
  (pad "K" smd rect (at -0.7875 0 336) (size 0.875 0.95) (layers "F.Cu" "F.Mask" "F.Paste") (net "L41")))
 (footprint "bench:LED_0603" (layer "F.Cu") (at 105.2191 149.1811 -84)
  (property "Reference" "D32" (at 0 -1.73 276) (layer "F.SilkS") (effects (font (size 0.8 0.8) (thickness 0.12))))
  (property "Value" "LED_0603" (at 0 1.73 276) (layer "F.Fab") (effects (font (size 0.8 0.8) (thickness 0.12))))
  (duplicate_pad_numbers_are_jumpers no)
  (pad "A" smd rect (at 0.7875 0 276) (size 0.875 0.95) (layers "F.Cu" "F.Mask" "F.Paste") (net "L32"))
  (pad "K" smd rect (at -0.7875 0 276) (size 0.875 0.95) (layers "F.Cu" "F.Mask" "F.Paste") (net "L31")))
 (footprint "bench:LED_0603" (layer "F.Cu") (at 128.7305 108.4582 -156)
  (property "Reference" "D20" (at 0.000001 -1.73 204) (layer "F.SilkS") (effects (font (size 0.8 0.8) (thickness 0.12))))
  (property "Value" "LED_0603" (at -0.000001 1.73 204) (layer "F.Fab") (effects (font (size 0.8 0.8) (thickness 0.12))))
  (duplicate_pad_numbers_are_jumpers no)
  (pad "A" smd rect (at 0.7875 0 204) (size 0.875 0.95) (layers "F.Cu" "F.Mask" "F.Paste") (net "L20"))
  (pad "K" smd rect (at -0.7875 0 204) (size 0.875 0.95) (layers "F.Cu" "F.Mask" "F.Paste") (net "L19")))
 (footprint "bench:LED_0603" (layer "F.Cu") (at 165 110.359 150)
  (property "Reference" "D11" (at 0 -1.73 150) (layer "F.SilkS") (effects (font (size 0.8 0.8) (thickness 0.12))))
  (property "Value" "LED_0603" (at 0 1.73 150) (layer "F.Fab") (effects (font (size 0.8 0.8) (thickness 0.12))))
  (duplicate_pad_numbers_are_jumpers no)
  (pad "A" smd rect (at 0.7875 0 150) (size 0.875 0.95) (layers "F.Cu" "F.Mask" "F.Paste") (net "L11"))
  (pad "K" smd rect (at -0.7875 0 150) (size 0.875 0.95) (layers "F.Cu" "F.Mask" "F.Paste") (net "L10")))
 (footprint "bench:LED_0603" (layer "F.Cu") (at 184.7809 149.1811 84)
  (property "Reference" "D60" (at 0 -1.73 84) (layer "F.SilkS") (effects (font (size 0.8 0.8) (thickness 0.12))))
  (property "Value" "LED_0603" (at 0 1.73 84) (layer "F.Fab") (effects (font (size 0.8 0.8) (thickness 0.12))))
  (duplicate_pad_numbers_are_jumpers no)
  (pad "A" smd rect (at 0.7875 0 84) (size 0.875 0.95) (layers "F.Cu" "F.Mask" "F.Paste") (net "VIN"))
  (pad "K" smd rect (at -0.7875 0 84) (size 0.875 0.95) (layers "F.Cu" "F.Mask" "F.Paste") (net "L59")))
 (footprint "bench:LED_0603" (layer "F.Cu") (at 161.2695 108.4582 156)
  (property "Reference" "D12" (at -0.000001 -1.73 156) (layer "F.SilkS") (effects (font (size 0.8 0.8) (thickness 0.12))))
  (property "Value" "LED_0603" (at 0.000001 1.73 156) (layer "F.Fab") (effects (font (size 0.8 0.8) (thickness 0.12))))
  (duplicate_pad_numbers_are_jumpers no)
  (pad "A" smd rect (at 0.7875 0 156) (size 0.875 0.95) (layers "F.Cu" "F.Mask" "F.Paste") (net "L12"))
  (pad "K" smd rect (at -0.7875 0 156) (size 0.875 0.95) (layers "F.Cu" "F.Mask" "F.Paste") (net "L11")))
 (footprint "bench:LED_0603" (layer "F.Cu") (at 108.4582 161.2695 -66)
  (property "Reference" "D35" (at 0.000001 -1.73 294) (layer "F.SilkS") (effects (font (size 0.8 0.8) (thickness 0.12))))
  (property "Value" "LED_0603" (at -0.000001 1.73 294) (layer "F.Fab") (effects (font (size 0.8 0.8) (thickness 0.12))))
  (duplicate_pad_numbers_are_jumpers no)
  (pad "A" smd rect (at 0.7875 0 294) (size 0.875 0.95) (layers "F.Cu" "F.Mask" "F.Paste") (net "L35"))
  (pad "K" smd rect (at -0.7875 0 294) (size 0.875 0.95) (layers "F.Cu" "F.Mask" "F.Paste") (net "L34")))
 (gr_line (start 100 100) (end 100 190) (stroke (width 0.1) (type solid)) (layer "Edge.Cuts"))
 (gr_line (start 100 190) (end 190 190) (stroke (width 0.1) (type solid)) (layer "Edge.Cuts"))
 (gr_line (start 190 100) (end 100 100) (stroke (width 0.1) (type solid)) (layer "Edge.Cuts"))
 (gr_line (start 190 190) (end 190 100) (stroke (width 0.1) (type solid)) (layer "Edge.Cuts"))
 (segment (start 143.7 145) (end 147.1 148.4) (width 0.15) (layer "F.Cu") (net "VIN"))
 (segment (start 147.1 148.4) (end 184.9 148.4) (width 0.15) (layer "F.Cu") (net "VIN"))
 (segment (start 147.1 145.8) (end 185 145.8) (width 0.15) (layer "F.Cu") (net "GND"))
 (segment (start 146.3 145) (end 147.1 145.8) (width 0.15) (layer "F.Cu") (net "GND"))
 (segment (start 184.9 144.1) (end 184.9 141.6) (width 0.15) (layer "F.Cu") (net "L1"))
 (segment (start 184.7 140) (end 184.3 139.6) (width 0.15) (layer "F.Cu") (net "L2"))
 (segment (start 184.3 139.6) (end 184.3 137.5) (width 0.15) (layer "F.Cu") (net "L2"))
 (segment (start 184 135.9) (end 183.3 135.2) (width 0.15) (layer "F.Cu") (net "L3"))
 (segment (start 183.3 135.2) (end 183.3 133.4) (width 0.15) (layer "F.Cu") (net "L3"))
 (segment (start 181.9 131) (end 181.9 129.4) (width 0.15) (layer "F.Cu") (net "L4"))
 (segment (start 182.8 131.9) (end 181.9 131) (width 0.15) (layer "F.Cu") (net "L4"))
 (segment (start 180 126.8) (end 180 125.7) (width 0.15) (layer "F.Cu") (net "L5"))
 (segment (start 181.2 128) (end 180 126.8) (width 0.15) (layer "F.Cu") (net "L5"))
 (segment (start 177.8 122.9) (end 177.8 122.1) (width 0.15) (layer "F.Cu") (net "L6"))
 (segment (start 179.2 124.3) (end 177.8 122.9) (width 0.15) (layer "F.Cu") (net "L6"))
 (segment (start 176.9 120.9) (end 175.3 119.3) (width 0.15) (layer "F.Cu") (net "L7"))
 (segment (start 174.2 117.6) (end 172.4 115.8) (width 0.15) (layer "F.Cu") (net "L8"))
 (segment (start 171.2 114.7) (end 169.6 113.1) (width 0.15) (layer "F.Cu") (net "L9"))
 (segment (start 166.5 110.8) (end 165.7 110.8) (width 0.15) (layer "F.Cu") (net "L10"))
 (segment (start 167.9 112.2) (end 166.5 110.8) (width 0.15) (layer "F.Cu") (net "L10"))
 (segment (start 164.3 110) (end 163.1 108.8) (width 0.15) (layer "F.Cu") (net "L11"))
 (segment (start 163.1 108.8) (end 162 108.8) (width 0.15) (layer "F.Cu") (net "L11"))
 (segment (start 160.6 108.1) (end 159.7 107.2) (width 0.15) (layer "F.Cu") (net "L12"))
 (segment (start 159.7 107.2) (end 158.1 107.2) (width 0.15) (layer "F.Cu") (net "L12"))
 (segment (start 156.6 106.7) (end 155.9 106) (width 0.15) (layer "F.Cu") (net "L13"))
 (segment (start 155.9 106) (end 154.1 106) (width 0.15) (layer "F.Cu") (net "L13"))
 (segment (start 152.1 105.3) (end 150 105.3) (width 0.15) (layer "F.Cu") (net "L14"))
 (segment (start 152.5 105.7) (end 152.1 105.3) (width 0.15) (layer "F.Cu") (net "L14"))
 (segment (start 148.3 105) (end 145.8 105) (width 0.15) (layer "F.Cu") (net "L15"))
 (segment (start 144.1 105.1) (end 141.6 105.1) (width 0.15) (layer "F.Cu") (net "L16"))
 (segment (start 140 105.3) (end 139.6 105.7) (width 0.15) (layer "F.Cu") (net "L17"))
 (segment (start 139.6 105.7) (end 137.5 105.7) (width 0.15) (layer "F.Cu") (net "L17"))
 (segment (start 135.9 106) (end 135.2 106.7) (width 0.15) (layer "F.Cu") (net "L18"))
 (segment (start 135.2 106.7) (end 133.4 106.7) (width 0.15) (layer "F.Cu") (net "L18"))
 (segment (start 131.9 107.2) (end 131 108.1) (width 0.15) (layer "F.Cu") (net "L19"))
 (segment (start 131 108.1) (end 129.4 108.1) (width 0.15) (layer "F.Cu") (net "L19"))
 (segment (start 126.8 110) (end 125.7 110) (width 0.15) (layer "F.Cu") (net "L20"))
 (segment (start 128 108.8) (end 126.8 110) (width 0.15) (layer "F.Cu") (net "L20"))
 (segment (start 122.9 112.2) (end 122.1 112.2) (width 0.15) (layer "F.Cu") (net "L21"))
 (segment (start 124.3 110.8) (end 122.9 112.2) (width 0.15) (layer "F.Cu") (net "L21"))
 (segment (start 120.9 113.1) (end 119.3 114.7) (width 0.15) (layer "F.Cu") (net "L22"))
 (segment (start 117.6 115.8) (end 115.8 117.6) (width 0.15) (layer "F.Cu") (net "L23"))
 (segment (start 114.7 118.8) (end 113.1 120.4) (width 0.15) (layer "F.Cu") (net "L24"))
 (segment (start 112.2 122.1) (end 110.8 123.5) (width 0.15) (layer "F.Cu") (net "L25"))
 (segment (start 110.8 123.5) (end 110.8 124.3) (width 0.15) (layer "F.Cu") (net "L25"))
 (segment (start 110 125.7) (end 108.8 126.9) (width 0.15) (layer "F.Cu") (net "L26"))
 (segment (start 108.8 126.9) (end 108.8 128) (width 0.15) (layer "F.Cu") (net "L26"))
 (segment (start 107.2 130.3) (end 107.2 131.9) (width 0.15) (layer "F.Cu") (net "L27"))
 (segment (start 108.1 129.4) (end 107.2 130.3) (width 0.15) (layer "F.Cu") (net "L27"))
 (segment (start 106 134.1) (end 106 135.9) (width 0.15) (layer "F.Cu") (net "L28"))
 (segment (start 106.7 133.4) (end 106 134.1) (width 0.15) (layer "F.Cu") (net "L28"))
 (segment (start 105.3 137.9) (end 105.3 140) (width 0.15) (layer "F.Cu") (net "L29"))
 (segment (start 105.7 137.5) (end 105.3 137.9) (width 0.15) (layer "F.Cu") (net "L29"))
 (segment (start 105 141.7) (end 105 144.2) (width 0.15) (layer "F.Cu") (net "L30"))
 (segment (start 105.1 145.9) (end 105.1 148.4) (width 0.15) (layer "F.Cu") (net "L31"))
 (segment (start 105.3 150) (end 105.7 150.4) (width 0.15) (layer "F.Cu") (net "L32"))
 (segment (start 105.7 150.4) (end 105.7 152.5) (width 0.15) (layer "F.Cu") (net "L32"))
 (segment (start 106.7 154.8) (end 106.7 156.6) (width 0.15) (layer "F.Cu") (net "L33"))
 (segment (start 106 154.1) (end 106.7 154.8) (width 0.15) (layer "F.Cu") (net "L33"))
 (segment (start 108.1 159) (end 108.1 160.6) (width 0.15) (layer "F.Cu") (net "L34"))
 (segment (start 107.2 158.1) (end 108.1 159) (width 0.15) (layer "F.Cu") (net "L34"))
 (segment (start 108.8 162) (end 110 163.2) (width 0.15) (layer "F.Cu") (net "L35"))
 (segment (start 110 163.2) (end 110 164.3) (width 0.15) (layer "F.Cu") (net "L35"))
 (segment (start 110.8 165.7) (end 112.2 167.1) (width 0.15) (layer "F.Cu") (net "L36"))
 (segment (start 112.2 167.1) (end 112.2 167.9) (width 0.15) (layer "F.Cu") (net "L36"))
 (segment (start 113.1 169.1) (end 114.7 170.7) (width 0.15) (layer "F.Cu") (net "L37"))
 (segment (start 115.8 172.4) (end 117.6 174.2) (width 0.15) (layer "F.Cu") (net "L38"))
 (segment (start 118.8 175.3) (end 120.4 176.9) (width 0.15) (layer "F.Cu") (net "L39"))
 (segment (start 123.5 179.2) (end 124.3 179.2) (width 0.15) (layer "F.Cu") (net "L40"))
 (segment (start 122.1 177.8) (end 123.5 179.2) (width 0.15) (layer "F.Cu") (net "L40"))
 (segment (start 126.9 181.2) (end 128 181.2) (width 0.15) (layer "F.Cu") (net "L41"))
 (segment (start 125.7 180) (end 126.9 181.2) (width 0.15) (layer "F.Cu") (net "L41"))
 (segment (start 129.4 181.9) (end 130.3 182.8) (width 0.15) (layer "F.Cu") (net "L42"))
 (segment (start 130.3 182.8) (end 131.9 182.8) (width 0.15) (layer "F.Cu") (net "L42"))
 (segment (start 133.4 183.3) (end 134.1 184) (width 0.15) (layer "F.Cu") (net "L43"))
 (segment (start 134.1 184) (end 135.9 184) (width 0.15) (layer "F.Cu") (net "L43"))
 (segment (start 137.5 184.3) (end 137.9 184.7) (width 0.15) (layer "F.Cu") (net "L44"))
 (segment (start 137.9 184.7) (end 140 184.7) (width 0.15) (layer "F.Cu") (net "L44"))
 (segment (start 141.7 185) (end 144.2 185) (width 0.15) (layer "F.Cu") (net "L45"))
 (segment (start 145.9 184.9) (end 148.4 184.9) (width 0.15) (layer "F.Cu") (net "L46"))
 (segment (start 150.4 184.3) (end 152.5 184.3) (width 0.15) (layer "F.Cu") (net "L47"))
 (segment (start 150 184.7) (end 150.4 184.3) (width 0.15) (layer "F.Cu") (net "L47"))
 (segment (start 154.1 184) (end 154.8 183.3) (width 0.15) (layer "F.Cu") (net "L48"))
 (segment (start 154.8 183.3) (end 156.6 183.3) (width 0.15) (layer "F.Cu") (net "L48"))
 (segment (start 159 181.9) (end 160.6 181.9) (width 0.15) (layer "F.Cu") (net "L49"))
 (segment (start 158.1 182.8) (end 159 181.9) (width 0.15) (layer "F.Cu") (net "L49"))
 (segment (start 162 181.2) (end 163.2 180) (width 0.15) (layer "F.Cu") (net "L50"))
 (segment (start 163.2 180) (end 164.3 180) (width 0.15) (layer "F.Cu") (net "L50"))
 (segment (start 167.1 177.8) (end 167.9 177.8) (width 0.15) (layer "F.Cu") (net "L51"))
 (segment (start 165.7 179.2) (end 167.1 177.8) (width 0.15) (layer "F.Cu") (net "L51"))
 (segment (start 169.1 176.9) (end 170.7 175.3) (width 0.15) (layer "F.Cu") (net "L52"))
 (segment (start 172.4 174.2) (end 174.2 172.4) (width 0.15) (layer "F.Cu") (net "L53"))
 (segment (start 175.3 171.2) (end 176.9 169.6) (width 0.15) (layer "F.Cu") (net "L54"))
 (segment (start 179.2 166.5) (end 179.2 165.7) (width 0.15) (layer "F.Cu") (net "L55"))
 (segment (start 177.8 167.9) (end 179.2 166.5) (width 0.15) (layer "F.Cu") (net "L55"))
 (segment (start 181.2 163.1) (end 181.2 162) (width 0.15) (layer "F.Cu") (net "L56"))
 (segment (start 180 164.3) (end 181.2 163.1) (width 0.15) (layer "F.Cu") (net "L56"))
 (segment (start 182.8 159.7) (end 182.8 158.1) (width 0.15) (layer "F.Cu") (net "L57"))
 (segment (start 181.9 160.6) (end 182.8 159.7) (width 0.15) (layer "F.Cu") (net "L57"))
 (segment (start 184 155.9) (end 184 154.1) (width 0.15) (layer "F.Cu") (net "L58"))
 (segment (start 183.3 156.6) (end 184 155.9) (width 0.15) (layer "F.Cu") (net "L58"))
 (segment (start 184.3 152.5) (end 184.7 152.1) (width 0.15) (layer "F.Cu") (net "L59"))
 (segment (start 184.7 152.1) (end 184.7 150) (width 0.15) (layer "F.Cu") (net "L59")))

